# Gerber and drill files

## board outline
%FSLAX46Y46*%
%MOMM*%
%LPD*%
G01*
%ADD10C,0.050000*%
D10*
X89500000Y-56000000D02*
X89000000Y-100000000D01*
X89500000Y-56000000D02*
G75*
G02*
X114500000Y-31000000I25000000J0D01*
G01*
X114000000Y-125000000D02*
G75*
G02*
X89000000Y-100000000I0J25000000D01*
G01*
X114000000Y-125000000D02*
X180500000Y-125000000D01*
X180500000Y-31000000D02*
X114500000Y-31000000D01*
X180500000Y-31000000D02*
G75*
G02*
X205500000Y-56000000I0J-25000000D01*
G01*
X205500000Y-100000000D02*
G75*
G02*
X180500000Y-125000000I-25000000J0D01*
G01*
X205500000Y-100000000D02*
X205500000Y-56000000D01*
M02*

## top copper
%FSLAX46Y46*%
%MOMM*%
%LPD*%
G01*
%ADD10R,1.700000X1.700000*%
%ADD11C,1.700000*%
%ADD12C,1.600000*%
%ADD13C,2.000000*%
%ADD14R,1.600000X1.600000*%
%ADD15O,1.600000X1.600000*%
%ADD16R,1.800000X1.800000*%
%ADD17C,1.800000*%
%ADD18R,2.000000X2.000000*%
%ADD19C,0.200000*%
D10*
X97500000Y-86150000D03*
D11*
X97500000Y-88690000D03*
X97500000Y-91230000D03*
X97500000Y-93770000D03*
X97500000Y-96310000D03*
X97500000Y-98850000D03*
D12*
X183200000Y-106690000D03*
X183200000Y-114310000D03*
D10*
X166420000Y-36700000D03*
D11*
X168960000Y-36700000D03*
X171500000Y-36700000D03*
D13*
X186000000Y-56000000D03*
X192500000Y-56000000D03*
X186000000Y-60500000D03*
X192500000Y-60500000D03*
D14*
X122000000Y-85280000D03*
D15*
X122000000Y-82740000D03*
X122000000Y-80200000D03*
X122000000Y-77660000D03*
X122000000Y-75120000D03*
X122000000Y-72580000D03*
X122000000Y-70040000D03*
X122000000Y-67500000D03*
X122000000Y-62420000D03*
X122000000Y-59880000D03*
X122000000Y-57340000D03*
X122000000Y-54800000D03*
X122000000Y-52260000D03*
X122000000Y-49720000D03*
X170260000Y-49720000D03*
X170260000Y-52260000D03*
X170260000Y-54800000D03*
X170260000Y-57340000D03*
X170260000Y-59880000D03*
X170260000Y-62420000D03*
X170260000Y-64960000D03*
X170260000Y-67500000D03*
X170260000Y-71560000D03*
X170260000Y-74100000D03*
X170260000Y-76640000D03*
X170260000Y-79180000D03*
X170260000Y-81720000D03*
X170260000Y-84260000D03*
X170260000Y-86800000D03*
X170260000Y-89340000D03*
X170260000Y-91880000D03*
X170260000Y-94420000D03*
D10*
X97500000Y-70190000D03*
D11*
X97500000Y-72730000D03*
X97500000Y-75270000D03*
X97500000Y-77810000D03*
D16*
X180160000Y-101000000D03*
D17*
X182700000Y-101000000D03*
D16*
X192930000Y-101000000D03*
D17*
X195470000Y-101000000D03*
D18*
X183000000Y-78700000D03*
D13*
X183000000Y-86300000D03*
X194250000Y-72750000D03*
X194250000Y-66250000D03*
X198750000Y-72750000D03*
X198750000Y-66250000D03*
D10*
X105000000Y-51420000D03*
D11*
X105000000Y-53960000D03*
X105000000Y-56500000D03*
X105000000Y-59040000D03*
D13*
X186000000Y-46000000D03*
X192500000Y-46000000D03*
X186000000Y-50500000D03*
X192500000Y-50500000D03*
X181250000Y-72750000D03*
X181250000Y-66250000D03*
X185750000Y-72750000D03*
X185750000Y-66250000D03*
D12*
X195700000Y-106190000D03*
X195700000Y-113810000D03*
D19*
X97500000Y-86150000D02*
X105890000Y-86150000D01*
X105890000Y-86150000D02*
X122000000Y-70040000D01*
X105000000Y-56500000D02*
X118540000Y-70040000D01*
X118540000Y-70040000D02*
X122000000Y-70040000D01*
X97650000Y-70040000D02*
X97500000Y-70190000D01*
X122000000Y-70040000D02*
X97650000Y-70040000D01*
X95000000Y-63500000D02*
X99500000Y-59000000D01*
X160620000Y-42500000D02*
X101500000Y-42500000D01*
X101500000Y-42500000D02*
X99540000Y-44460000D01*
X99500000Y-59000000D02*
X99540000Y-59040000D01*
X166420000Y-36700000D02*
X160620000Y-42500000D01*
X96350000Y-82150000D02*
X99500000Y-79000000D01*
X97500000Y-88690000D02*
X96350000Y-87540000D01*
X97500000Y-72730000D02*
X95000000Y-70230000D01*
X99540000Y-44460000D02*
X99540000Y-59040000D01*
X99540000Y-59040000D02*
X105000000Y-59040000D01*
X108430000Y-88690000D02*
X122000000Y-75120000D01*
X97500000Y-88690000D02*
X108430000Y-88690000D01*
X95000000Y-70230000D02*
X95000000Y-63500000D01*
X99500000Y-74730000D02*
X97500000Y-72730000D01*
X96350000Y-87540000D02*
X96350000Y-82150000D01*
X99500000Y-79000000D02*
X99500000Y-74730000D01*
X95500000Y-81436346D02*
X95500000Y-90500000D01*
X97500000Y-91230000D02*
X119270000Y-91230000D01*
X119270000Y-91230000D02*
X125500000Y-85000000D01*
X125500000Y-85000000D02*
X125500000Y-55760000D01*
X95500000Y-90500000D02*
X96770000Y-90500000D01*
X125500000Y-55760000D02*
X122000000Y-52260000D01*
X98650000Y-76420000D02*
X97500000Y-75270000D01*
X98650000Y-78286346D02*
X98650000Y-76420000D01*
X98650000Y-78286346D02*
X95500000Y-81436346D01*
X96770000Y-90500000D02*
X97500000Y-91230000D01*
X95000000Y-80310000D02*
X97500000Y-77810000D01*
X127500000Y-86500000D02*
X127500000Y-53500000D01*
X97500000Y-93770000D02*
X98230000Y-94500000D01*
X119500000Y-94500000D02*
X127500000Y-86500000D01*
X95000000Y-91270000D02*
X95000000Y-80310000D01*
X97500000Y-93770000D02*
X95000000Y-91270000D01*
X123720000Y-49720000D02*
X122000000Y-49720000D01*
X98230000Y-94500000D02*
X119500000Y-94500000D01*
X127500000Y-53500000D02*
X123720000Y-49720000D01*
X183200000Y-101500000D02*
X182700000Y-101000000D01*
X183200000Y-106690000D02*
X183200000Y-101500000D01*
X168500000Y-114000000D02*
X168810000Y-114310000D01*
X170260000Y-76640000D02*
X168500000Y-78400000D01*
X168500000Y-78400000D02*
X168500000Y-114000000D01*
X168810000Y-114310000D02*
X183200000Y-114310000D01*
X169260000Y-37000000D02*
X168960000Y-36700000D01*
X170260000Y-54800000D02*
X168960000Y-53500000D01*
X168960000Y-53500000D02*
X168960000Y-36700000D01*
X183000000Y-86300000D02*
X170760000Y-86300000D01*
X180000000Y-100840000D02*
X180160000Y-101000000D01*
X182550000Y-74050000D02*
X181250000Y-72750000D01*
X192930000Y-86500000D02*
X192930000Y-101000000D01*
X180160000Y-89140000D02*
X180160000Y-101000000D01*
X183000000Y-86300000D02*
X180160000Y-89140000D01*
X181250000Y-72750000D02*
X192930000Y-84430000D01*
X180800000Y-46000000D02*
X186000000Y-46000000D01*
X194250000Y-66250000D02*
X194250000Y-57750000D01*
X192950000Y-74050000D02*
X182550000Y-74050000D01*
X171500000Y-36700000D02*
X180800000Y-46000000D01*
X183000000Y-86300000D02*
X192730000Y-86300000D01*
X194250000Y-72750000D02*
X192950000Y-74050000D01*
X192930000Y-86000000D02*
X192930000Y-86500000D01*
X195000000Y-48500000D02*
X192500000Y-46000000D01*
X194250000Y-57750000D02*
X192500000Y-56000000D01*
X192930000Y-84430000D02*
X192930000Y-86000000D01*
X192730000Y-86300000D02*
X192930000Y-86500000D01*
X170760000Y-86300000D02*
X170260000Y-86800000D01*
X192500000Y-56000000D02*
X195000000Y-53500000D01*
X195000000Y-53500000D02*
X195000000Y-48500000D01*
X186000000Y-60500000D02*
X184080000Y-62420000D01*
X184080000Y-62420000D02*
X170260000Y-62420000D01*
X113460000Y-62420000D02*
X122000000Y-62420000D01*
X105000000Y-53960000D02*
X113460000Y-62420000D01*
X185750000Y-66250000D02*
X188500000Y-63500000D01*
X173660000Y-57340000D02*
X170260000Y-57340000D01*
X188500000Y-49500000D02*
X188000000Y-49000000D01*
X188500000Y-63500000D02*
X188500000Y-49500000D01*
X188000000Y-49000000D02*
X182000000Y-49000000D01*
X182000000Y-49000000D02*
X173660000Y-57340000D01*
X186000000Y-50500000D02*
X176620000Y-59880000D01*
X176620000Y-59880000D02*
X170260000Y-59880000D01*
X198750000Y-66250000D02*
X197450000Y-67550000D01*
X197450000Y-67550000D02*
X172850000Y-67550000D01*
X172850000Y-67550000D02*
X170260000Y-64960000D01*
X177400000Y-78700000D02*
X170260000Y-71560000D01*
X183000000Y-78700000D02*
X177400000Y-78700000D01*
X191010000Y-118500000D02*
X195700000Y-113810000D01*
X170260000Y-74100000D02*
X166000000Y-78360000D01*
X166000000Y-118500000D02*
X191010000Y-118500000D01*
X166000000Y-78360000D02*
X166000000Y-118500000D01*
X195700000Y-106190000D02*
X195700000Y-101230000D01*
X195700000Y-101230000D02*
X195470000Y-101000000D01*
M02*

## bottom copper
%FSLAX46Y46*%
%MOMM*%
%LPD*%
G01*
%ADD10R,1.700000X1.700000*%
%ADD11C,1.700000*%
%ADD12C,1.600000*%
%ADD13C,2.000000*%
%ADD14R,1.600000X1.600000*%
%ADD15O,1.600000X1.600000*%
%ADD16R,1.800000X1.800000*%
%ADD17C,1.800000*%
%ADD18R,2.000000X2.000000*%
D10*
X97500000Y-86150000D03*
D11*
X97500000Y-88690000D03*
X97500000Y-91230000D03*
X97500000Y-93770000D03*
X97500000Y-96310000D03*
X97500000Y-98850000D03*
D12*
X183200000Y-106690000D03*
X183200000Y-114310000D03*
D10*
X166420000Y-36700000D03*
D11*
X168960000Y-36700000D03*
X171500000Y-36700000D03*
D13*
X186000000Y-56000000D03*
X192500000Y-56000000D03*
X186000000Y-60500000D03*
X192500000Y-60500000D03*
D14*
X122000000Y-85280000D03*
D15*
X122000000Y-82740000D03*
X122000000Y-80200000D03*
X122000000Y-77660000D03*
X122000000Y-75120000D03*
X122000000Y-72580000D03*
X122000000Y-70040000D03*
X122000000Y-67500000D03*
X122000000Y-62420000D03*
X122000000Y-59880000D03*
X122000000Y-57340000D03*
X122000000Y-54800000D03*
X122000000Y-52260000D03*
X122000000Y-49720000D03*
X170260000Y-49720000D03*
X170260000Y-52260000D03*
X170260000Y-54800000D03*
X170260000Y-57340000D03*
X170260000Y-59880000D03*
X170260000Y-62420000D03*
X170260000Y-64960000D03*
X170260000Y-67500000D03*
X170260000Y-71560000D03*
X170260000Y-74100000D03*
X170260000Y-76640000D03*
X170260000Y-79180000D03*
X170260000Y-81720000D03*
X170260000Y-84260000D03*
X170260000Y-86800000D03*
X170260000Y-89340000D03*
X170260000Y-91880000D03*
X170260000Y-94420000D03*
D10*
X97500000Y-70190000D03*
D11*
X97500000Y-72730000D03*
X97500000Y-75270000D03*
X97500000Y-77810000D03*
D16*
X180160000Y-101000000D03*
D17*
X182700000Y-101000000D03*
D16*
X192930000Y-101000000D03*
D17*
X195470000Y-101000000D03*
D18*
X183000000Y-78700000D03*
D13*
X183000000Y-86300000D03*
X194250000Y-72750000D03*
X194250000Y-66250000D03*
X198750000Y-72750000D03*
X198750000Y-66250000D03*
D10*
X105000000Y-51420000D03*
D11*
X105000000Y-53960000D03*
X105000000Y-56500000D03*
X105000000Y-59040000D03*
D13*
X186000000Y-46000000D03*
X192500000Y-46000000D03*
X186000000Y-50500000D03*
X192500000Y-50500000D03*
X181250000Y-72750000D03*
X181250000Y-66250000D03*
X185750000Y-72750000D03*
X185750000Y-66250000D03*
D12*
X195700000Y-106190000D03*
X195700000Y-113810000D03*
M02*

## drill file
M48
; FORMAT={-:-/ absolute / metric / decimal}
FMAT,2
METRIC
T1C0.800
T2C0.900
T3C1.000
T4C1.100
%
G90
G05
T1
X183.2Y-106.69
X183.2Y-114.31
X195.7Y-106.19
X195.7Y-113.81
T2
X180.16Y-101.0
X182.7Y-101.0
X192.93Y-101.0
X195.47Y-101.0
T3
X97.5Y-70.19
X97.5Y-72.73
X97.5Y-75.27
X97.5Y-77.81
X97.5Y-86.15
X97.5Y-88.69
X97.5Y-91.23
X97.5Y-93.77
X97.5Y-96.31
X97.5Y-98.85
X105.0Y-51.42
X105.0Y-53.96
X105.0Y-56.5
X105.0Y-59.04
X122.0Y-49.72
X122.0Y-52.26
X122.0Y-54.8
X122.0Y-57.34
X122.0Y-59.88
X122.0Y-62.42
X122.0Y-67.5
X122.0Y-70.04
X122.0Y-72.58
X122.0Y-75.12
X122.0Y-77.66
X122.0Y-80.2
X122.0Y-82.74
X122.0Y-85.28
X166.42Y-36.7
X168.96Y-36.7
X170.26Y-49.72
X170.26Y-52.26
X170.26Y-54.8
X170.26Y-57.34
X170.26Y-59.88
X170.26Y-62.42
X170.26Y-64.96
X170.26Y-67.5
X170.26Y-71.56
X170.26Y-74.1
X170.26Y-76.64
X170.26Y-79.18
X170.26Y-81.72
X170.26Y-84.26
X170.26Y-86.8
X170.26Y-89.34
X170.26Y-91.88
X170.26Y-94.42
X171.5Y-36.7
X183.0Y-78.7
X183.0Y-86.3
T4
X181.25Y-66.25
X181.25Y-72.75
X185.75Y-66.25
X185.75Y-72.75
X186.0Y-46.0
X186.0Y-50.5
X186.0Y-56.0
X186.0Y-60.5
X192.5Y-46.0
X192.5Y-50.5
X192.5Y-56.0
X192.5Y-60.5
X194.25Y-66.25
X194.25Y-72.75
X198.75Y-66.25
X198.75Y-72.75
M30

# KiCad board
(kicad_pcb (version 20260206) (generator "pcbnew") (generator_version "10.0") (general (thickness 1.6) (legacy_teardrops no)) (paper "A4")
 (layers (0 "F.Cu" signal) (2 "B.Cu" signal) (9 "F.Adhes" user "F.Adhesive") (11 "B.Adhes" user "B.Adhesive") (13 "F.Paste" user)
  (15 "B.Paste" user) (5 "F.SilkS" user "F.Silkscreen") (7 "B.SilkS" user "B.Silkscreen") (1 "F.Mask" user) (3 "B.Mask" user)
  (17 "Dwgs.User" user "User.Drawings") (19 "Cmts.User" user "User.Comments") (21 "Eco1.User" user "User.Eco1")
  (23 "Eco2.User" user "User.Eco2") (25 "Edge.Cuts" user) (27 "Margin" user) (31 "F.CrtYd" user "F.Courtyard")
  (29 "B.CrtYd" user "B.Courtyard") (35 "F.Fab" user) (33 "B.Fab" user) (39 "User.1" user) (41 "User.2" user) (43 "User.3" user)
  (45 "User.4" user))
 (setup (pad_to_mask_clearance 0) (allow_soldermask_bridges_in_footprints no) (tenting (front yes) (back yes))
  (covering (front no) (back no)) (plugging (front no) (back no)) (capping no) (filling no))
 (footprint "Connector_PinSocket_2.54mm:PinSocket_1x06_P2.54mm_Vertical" (layer "F.Cu") (at 97.5 86.15)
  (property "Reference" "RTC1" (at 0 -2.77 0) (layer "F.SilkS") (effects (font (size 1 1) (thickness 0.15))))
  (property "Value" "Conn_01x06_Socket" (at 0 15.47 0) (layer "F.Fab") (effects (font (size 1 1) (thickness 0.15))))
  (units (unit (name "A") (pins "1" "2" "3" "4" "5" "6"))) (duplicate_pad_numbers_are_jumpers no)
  (pad "1" thru_hole rect (at 0 0) (size 1.7 1.7) (drill 1) (layers "*.Cu" "*.Mask") (remove_unused_layers no) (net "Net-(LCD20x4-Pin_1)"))
  (pad "2" thru_hole circle (at 0 2.54) (size 1.7 1.7) (drill 1) (layers "*.Cu" "*.Mask") (remove_unused_layers no) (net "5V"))
  (pad "3" thru_hole circle (at 0 5.08) (size 1.7 1.7) (drill 1) (layers "*.Cu" "*.Mask") (remove_unused_layers no)
   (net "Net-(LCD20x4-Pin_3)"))
  (pad "4" thru_hole circle (at 0 7.62) (size 1.7 1.7) (drill 1) (layers "*.Cu" "*.Mask") (remove_unused_layers no)
   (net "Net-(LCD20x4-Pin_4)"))
  (pad "5" thru_hole circle (at 0 10.16) (size 1.7 1.7) (drill 1) (layers "*.Cu" "*.Mask") (remove_unused_layers no)
   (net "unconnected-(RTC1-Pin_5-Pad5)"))
  (pad "6" thru_hole circle (at 0 12.7) (size 1.7 1.7) (drill 1) (layers "*.Cu" "*.Mask") (remove_unused_layers no)
   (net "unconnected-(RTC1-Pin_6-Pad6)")))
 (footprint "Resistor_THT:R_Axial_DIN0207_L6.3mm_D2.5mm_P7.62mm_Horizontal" (layer "F.Cu") (at 183.2 106.69 -90)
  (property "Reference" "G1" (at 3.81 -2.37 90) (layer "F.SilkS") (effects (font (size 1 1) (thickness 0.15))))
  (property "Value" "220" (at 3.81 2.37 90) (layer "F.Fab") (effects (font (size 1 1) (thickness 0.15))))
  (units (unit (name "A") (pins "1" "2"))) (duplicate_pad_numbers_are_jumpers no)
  (pad "1" thru_hole circle (at 0 0 270) (size 1.6 1.6) (drill 0.8) (layers "*.Cu" "*.Mask") (remove_unused_layers no)
   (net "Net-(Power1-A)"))
  (pad "2" thru_hole circle (at 7.62 0 270) (size 1.6 1.6) (drill 0.8) (layers "*.Cu" "*.Mask") (remove_unused_layers no)
   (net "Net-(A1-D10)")))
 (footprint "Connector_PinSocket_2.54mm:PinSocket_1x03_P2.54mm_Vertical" (layer "F.Cu") (at 166.42 36.7 90)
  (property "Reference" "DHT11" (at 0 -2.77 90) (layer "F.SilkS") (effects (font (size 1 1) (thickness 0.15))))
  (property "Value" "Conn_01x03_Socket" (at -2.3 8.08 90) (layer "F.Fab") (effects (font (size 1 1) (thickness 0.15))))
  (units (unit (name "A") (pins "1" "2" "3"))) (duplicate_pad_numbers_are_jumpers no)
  (pad "1" thru_hole rect (at 0 0 90) (size 1.7 1.7) (drill 1) (layers "*.Cu" "*.Mask") (remove_unused_layers no) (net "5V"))
  (pad "2" thru_hole circle (at 0 2.54 90) (size 1.7 1.7) (drill 1) (layers "*.Cu" "*.Mask") (remove_unused_layers no) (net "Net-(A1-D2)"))
  (pad "3" thru_hole circle (at 0 5.08 90) (size 1.7 1.7) (drill 1) (layers "*.Cu" "*.Mask") (remove_unused_layers no)
   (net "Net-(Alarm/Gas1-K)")))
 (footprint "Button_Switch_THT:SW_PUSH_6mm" (layer "F.Cu") (at 186 56)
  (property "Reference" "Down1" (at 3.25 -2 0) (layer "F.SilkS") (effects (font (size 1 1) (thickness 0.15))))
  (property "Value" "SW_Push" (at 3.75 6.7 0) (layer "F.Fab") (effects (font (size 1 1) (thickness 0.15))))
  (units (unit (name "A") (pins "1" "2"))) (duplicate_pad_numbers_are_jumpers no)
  (pad "1" thru_hole circle (at 0 0 90) (size 2 2) (drill 1.1) (layers "*.Cu" "*.Mask") (remove_unused_layers no) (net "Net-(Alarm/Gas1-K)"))
  (pad "1" thru_hole circle (at 6.5 0 90) (size 2 2) (drill 1.1) (layers "*.Cu" "*.Mask") (remove_unused_layers no)
   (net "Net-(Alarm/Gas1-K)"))
  (pad "2" thru_hole circle (at 0 4.5 90) (size 2 2) (drill 1.1) (layers "*.Cu" "*.Mask") (remove_unused_layers no) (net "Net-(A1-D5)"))
  (pad "2" thru_hole circle (at 6.5 4.5 90) (size 2 2) (drill 1.1) (layers "*.Cu" "*.Mask") (remove_unused_layers no) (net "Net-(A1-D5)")))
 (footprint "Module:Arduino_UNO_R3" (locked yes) (layer "F.Cu") (at 122 85.28 90)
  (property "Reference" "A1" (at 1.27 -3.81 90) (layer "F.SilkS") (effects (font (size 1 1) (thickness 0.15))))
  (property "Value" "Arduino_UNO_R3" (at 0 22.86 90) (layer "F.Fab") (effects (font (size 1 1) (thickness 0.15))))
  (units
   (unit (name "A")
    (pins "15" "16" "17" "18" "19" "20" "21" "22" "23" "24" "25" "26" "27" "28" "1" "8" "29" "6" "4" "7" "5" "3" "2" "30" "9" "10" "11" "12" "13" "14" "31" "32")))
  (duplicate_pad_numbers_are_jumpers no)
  (pad "1" thru_hole rect (at 0 0 180) (size 1.6 1.6) (drill 1) (layers "*.Cu" "*.Mask") (remove_unused_layers no)
   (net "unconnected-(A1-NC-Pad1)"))
  (pad "2" thru_hole oval (at 2.54 0 180) (size 1.6 1.6) (drill 1) (layers "*.Cu" "*.Mask") (remove_unused_layers no)
   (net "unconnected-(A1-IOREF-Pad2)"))
  (pad "3" thru_hole oval (at 5.08 0 180) (size 1.6 1.6) (drill 1) (layers "*.Cu" "*.Mask") (remove_unused_layers no)
   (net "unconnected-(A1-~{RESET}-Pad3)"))
  (pad "4" thru_hole oval (at 7.62 0 180) (size 1.6 1.6) (drill 1) (layers "*.Cu" "*.Mask") (remove_unused_layers no)
   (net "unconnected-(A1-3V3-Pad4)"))
  (pad "5" thru_hole oval (at 10.16 0 180) (size 1.6 1.6) (drill 1) (layers "*.Cu" "*.Mask") (remove_unused_layers no) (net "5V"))
  (pad "6" thru_hole oval (at 12.7 0 180) (size 1.6 1.6) (drill 1) (layers "*.Cu" "*.Mask") (remove_unused_layers no) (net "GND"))
  (pad "7" thru_hole oval (at 15.24 0 180) (size 1.6 1.6) (drill 1) (layers "*.Cu" "*.Mask") (remove_unused_layers no)
   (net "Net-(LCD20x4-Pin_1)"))
  (pad "8" thru_hole oval (at 17.78 0 180) (size 1.6 1.6) (drill 1) (layers "*.Cu" "*.Mask") (remove_unused_layers no)
   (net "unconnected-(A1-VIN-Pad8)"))
  (pad "9" thru_hole oval (at 22.86 0 180) (size 1.6 1.6) (drill 1) (layers "*.Cu" "*.Mask") (remove_unused_layers no) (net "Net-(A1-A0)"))
  (pad "10" thru_hole oval (at 25.4 0 180) (size 1.6 1.6) (drill 1) (layers "*.Cu" "*.Mask") (remove_unused_layers no)
   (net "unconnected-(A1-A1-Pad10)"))
  (pad "11" thru_hole oval (at 27.94 0 180) (size 1.6 1.6) (drill 1) (layers "*.Cu" "*.Mask") (remove_unused_layers no)
   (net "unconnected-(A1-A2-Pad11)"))
  (pad "12" thru_hole oval (at 30.48 0 180) (size 1.6 1.6) (drill 1) (layers "*.Cu" "*.Mask") (remove_unused_layers no)
   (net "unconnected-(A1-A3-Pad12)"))
  (pad "13" thru_hole oval (at 33.02 0 180) (size 1.6 1.6) (drill 1) (layers "*.Cu" "*.Mask") (remove_unused_layers no)
   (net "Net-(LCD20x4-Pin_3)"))
  (pad "14" thru_hole oval (at 35.56 0 180) (size 1.6 1.6) (drill 1) (layers "*.Cu" "*.Mask") (remove_unused_layers no)
   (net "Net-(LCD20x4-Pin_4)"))
  (pad "15" thru_hole oval (at 35.56 48.26 180) (size 1.6 1.6) (drill 1) (layers "*.Cu" "*.Mask") (remove_unused_layers no)
   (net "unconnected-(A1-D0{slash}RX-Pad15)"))
  (pad "16" thru_hole oval (at 33.02 48.26 180) (size 1.6 1.6) (drill 1) (layers "*.Cu" "*.Mask") (remove_unused_layers no)
   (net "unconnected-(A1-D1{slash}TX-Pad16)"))
  (pad "17" thru_hole oval (at 30.48 48.26 180) (size 1.6 1.6) (drill 1) (layers "*.Cu" "*.Mask") (remove_unused_layers no)
   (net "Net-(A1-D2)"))
  (pad "18" thru_hole oval (at 27.94 48.26 180) (size 1.6 1.6) (drill 1) (layers "*.Cu" "*.Mask") (remove_unused_layers no)
   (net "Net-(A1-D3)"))
  (pad "19" thru_hole oval (at 25.4 48.26 180) (size 1.6 1.6) (drill 1) (layers "*.Cu" "*.Mask") (remove_unused_layers no)
   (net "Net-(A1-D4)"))
  (pad "20" thru_hole oval (at 22.86 48.26 180) (size 1.6 1.6) (drill 1) (layers "*.Cu" "*.Mask") (remove_unused_layers no)
   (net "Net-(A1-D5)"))
  (pad "21" thru_hole oval (at 20.32 48.26 180) (size 1.6 1.6) (drill 1) (layers "*.Cu" "*.Mask") (remove_unused_layers no)
   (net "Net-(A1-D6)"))
  (pad "22" thru_hole oval (at 17.78 48.26 180) (size 1.6 1.6) (drill 1) (layers "*.Cu" "*.Mask") (remove_unused_layers no)
   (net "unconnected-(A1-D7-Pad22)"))
  (pad "23" thru_hole oval (at 13.72 48.26 180) (size 1.6 1.6) (drill 1) (layers "*.Cu" "*.Mask") (remove_unused_layers no)
   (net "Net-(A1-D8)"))
  (pad "24" thru_hole oval (at 11.18 48.26 180) (size 1.6 1.6) (drill 1) (layers "*.Cu" "*.Mask") (remove_unused_layers no)
   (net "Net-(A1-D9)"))
  (pad "25" thru_hole oval (at 8.64 48.26 180) (size 1.6 1.6) (drill 1) (layers "*.Cu" "*.Mask") (remove_unused_layers no)
   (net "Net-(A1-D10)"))
  (pad "26" thru_hole oval (at 6.1 48.26 180) (size 1.6 1.6) (drill 1) (layers "*.Cu" "*.Mask") (remove_unused_layers no)
   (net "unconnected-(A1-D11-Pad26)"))
  (pad "27" thru_hole oval (at 3.56 48.26 180) (size 1.6 1.6) (drill 1) (layers "*.Cu" "*.Mask") (remove_unused_layers no)
   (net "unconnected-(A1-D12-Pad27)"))
  (pad "28" thru_hole oval (at 1.02 48.26 180) (size 1.6 1.6) (drill 1) (layers "*.Cu" "*.Mask") (remove_unused_layers no)
   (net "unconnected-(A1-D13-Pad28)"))
  (pad "29" thru_hole oval (at -1.52 48.26 180) (size 1.6 1.6) (drill 1) (layers "*.Cu" "*.Mask") (remove_unused_layers no)
   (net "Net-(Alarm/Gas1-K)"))
  (pad "30" thru_hole oval (at -4.06 48.26 180) (size 1.6 1.6) (drill 1) (layers "*.Cu" "*.Mask") (remove_unused_layers no)
   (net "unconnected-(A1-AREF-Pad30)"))
  (pad "31" thru_hole oval (at -6.6 48.26 180) (size 1.6 1.6) (drill 1) (layers "*.Cu" "*.Mask") (remove_unused_layers no)
   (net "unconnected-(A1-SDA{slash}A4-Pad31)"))
  (pad "32" thru_hole oval (at -9.14 48.26 180) (size 1.6 1.6) (drill 1) (layers "*.Cu" "*.Mask") (remove_unused_layers no)
   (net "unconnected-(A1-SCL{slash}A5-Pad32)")))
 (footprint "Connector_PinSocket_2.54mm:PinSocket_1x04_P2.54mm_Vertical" (layer "F.Cu") (at 97.5 70.19)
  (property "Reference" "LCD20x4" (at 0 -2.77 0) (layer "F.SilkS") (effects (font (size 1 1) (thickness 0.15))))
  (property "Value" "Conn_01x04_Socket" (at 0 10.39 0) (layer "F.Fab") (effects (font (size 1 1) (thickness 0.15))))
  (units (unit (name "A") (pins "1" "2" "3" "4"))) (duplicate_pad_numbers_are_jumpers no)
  (pad "1" thru_hole rect (at 0 0) (size 1.7 1.7) (drill 1) (layers "*.Cu" "*.Mask") (remove_unused_layers no) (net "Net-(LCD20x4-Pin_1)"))
  (pad "2" thru_hole circle (at 0 2.54) (size 1.7 1.7) (drill 1) (layers "*.Cu" "*.Mask") (remove_unused_layers no) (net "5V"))
  (pad "3" thru_hole circle (at 0 5.08) (size 1.7 1.7) (drill 1) (layers "*.Cu" "*.Mask") (remove_unused_layers no)
   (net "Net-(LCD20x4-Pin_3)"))
  (pad "4" thru_hole circle (at 0 7.62) (size 1.7 1.7) (drill 1) (layers "*.Cu" "*.Mask") (remove_unused_layers no)
   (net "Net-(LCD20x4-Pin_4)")))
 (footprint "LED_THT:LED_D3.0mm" (layer "F.Cu") (at 180.16 101)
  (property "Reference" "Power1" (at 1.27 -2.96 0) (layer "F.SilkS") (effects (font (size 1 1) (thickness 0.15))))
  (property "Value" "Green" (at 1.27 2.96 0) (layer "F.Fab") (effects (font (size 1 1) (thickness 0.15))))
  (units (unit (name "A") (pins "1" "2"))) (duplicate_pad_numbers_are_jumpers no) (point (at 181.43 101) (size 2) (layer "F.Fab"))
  (pad "1" thru_hole rect (at 0 0) (size 1.8 1.8) (drill 0.9) (layers "*.Cu" "*.Mask") (remove_unused_layers no) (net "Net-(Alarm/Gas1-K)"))
  (pad "2" thru_hole circle (at 2.54 0) (size 1.8 1.8) (drill 0.9) (layers "*.Cu" "*.Mask") (remove_unused_layers no) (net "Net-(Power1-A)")))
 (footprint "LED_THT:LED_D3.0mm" (layer "F.Cu") (at 192.93 101)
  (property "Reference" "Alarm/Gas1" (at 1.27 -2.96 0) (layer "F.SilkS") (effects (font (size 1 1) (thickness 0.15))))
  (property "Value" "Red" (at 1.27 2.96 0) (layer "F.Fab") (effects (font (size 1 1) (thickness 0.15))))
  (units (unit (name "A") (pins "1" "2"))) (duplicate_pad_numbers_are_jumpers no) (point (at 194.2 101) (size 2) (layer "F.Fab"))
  (pad "1" thru_hole rect (at 0 0) (size 1.8 1.8) (drill 0.9) (layers "*.Cu" "*.Mask") (remove_unused_layers no) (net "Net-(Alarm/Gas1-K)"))
  (pad "2" thru_hole circle (at 2.54 0) (size 1.8 1.8) (drill 0.9) (layers "*.Cu" "*.Mask") (remove_unused_layers no)
   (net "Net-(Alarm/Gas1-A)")))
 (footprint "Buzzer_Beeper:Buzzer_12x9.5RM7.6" (layer "F.Cu") (at 183 78.7 -90)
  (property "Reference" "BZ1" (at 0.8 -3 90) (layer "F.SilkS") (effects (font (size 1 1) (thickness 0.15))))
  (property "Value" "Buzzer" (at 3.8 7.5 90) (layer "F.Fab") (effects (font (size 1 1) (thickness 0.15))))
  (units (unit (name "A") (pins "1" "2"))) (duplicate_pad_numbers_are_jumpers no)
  (pad "1" thru_hole rect (at 0 0 270) (size 2 2) (drill 1) (layers "*.Cu" "*.Mask") (remove_unused_layers no) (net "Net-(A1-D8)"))
  (pad "2" thru_hole circle (at 7.6 0 270) (size 2 2) (drill 1) (layers "*.Cu" "*.Mask") (remove_unused_layers no)
   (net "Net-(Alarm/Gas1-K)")))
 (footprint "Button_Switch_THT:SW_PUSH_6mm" (layer "F.Cu") (at 194.25 72.75 90)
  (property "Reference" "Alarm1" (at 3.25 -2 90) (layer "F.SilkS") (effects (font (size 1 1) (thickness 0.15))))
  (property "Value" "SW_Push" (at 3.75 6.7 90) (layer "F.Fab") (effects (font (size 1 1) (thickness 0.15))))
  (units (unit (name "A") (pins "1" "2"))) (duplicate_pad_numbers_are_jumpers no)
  (pad "1" thru_hole circle (at 0 0 180) (size 2 2) (drill 1.1) (layers "*.Cu" "*.Mask") (remove_unused_layers no)
   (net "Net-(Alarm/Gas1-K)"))
  (pad "1" thru_hole circle (at 6.5 0 180) (size 2 2) (drill 1.1) (layers "*.Cu" "*.Mask") (remove_unused_layers no)
   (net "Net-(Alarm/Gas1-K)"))
  (pad "2" thru_hole circle (at 0 4.5 180) (size 2 2) (drill 1.1) (layers "*.Cu" "*.Mask") (remove_unused_layers no) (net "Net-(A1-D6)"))
  (pad "2" thru_hole circle (at 6.5 4.5 180) (size 2 2) (drill 1.1) (layers "*.Cu" "*.Mask") (remove_unused_layers no) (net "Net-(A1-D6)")))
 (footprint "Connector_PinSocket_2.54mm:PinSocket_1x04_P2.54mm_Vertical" (layer "F.Cu") (at 105 51.42)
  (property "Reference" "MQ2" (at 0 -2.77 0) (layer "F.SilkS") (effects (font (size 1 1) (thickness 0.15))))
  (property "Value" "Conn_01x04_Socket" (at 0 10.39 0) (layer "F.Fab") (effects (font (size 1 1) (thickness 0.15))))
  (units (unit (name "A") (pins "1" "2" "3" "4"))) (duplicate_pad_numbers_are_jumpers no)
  (pad "1" thru_hole rect (at 0 0) (size 1.7 1.7) (drill 1) (layers "*.Cu" "*.Mask") (remove_unused_layers no)
   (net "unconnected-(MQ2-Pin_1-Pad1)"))
  (pad "2" thru_hole circle (at 0 2.54) (size 1.7 1.7) (drill 1) (layers "*.Cu" "*.Mask") (remove_unused_layers no) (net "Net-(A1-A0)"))
  (pad "3" thru_hole circle (at 0 5.08) (size 1.7 1.7) (drill 1) (layers "*.Cu" "*.Mask") (remove_unused_layers no)
   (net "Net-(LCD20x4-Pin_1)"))
  (pad "4" thru_hole circle (at 0 7.62) (size 1.7 1.7) (drill 1) (layers "*.Cu" "*.Mask") (remove_unused_layers no) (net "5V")))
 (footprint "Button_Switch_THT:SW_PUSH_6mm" (layer "F.Cu") (at 186 46)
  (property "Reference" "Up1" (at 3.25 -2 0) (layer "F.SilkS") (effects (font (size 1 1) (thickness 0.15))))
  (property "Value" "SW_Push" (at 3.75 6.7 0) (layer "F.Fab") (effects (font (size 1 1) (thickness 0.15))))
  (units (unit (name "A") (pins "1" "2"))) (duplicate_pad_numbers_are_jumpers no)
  (pad "1" thru_hole circle (at 0 0 90) (size 2 2) (drill 1.1) (layers "*.Cu" "*.Mask") (remove_unused_layers no) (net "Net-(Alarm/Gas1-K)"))
  (pad "1" thru_hole circle (at 6.5 0 90) (size 2 2) (drill 1.1) (layers "*.Cu" "*.Mask") (remove_unused_layers no)
   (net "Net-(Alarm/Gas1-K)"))
  (pad "2" thru_hole circle (at 0 4.5 90) (size 2 2) (drill 1.1) (layers "*.Cu" "*.Mask") (remove_unused_layers no) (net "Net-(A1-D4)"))
  (pad "2" thru_hole circle (at 6.5 4.5 90) (size 2 2) (drill 1.1) (layers "*.Cu" "*.Mask") (remove_unused_layers no) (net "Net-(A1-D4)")))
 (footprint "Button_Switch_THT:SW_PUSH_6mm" (layer "F.Cu") (at 181.25 72.75 90)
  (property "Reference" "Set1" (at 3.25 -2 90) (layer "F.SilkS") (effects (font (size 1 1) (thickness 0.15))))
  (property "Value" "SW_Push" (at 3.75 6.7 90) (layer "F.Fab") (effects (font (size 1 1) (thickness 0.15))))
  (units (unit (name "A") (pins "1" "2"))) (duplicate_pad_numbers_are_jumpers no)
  (pad "1" thru_hole circle (at 0 0 180) (size 2 2) (drill 1.1) (layers "*.Cu" "*.Mask") (remove_unused_layers no)
   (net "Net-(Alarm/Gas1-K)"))
  (pad "1" thru_hole circle (at 6.5 0 180) (size 2 2) (drill 1.1) (layers "*.Cu" "*.Mask") (remove_unused_layers no)
   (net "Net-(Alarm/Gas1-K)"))
  (pad "2" thru_hole circle (at 0 4.5 180) (size 2 2) (drill 1.1) (layers "*.Cu" "*.Mask") (remove_unused_layers no) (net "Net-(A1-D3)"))
  (pad "2" thru_hole circle (at 6.5 4.5 180) (size 2 2) (drill 1.1) (layers "*.Cu" "*.Mask") (remove_unused_layers no) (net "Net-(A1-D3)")))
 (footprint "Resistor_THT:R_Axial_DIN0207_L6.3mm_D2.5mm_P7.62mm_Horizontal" (layer "F.Cu") (at 195.7 106.19 -90)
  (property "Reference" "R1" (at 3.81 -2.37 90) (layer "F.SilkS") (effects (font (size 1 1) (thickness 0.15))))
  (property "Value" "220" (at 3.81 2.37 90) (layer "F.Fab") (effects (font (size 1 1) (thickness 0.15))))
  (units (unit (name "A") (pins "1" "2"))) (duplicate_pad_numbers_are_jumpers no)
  (pad "1" thru_hole circle (at 0 0 270) (size 1.6 1.6) (drill 0.8) (layers "*.Cu" "*.Mask") (remove_unused_layers no)
   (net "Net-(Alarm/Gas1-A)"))
  (pad "2" thru_hole circle (at 7.62 0 270) (size 1.6 1.6) (drill 0.8) (layers "*.Cu" "*.Mask") (remove_unused_layers no)
   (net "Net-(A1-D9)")))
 (gr_line (start 89.5 56) (end 89 100) (stroke (width 0.05) (type default)) (layer "Edge.Cuts"))
 (gr_arc (start 89.5 56) (mid 96.82233 38.32233) (end 114.5 31) (stroke (width 0.05) (type default)) (layer "Edge.Cuts"))
 (gr_arc (start 114 125) (mid 96.32233 117.67767) (end 89 100) (stroke (width 0.05) (type default)) (layer "Edge.Cuts"))
 (gr_line (start 114 125) (end 180.5 125) (stroke (width 0.05) (type default)) (layer "Edge.Cuts"))
 (gr_line (start 180.5 31) (end 114.5 31) (stroke (width 0.05) (type default)) (layer "Edge.Cuts"))
 (gr_arc (start 180.5 31) (mid 198.17767 38.32233) (end 205.5 56) (stroke (width 0.05) (type default)) (layer "Edge.Cuts"))
 (gr_arc (start 205.5 100) (mid 198.17767 117.67767) (end 180.5 125) (stroke (width 0.05) (type default)) (layer "Edge.Cuts"))
 (gr_line (start 205.5 100) (end 205.5 56) (stroke (width 0.05) (type default)) (layer "Edge.Cuts"))
 (segment (start 97.5 86.15) (end 105.89 86.15) (width 0.2) (layer "F.Cu") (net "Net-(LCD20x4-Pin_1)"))
 (segment (start 105.89 86.15) (end 122 70.04) (width 0.2) (layer "F.Cu") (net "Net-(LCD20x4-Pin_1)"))
 (segment (start 105 56.5) (end 118.54 70.04) (width 0.2) (layer "F.Cu") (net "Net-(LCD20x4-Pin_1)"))
 (segment (start 118.54 70.04) (end 122 70.04) (width 0.2) (layer "F.Cu") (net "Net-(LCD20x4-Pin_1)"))
 (segment (start 97.65 70.04) (end 97.5 70.19) (width 0.2) (layer "F.Cu") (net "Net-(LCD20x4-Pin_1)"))
 (segment (start 122 70.04) (end 97.65 70.04) (width 0.2) (layer "F.Cu") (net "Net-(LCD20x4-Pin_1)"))
 (segment (start 95 63.5) (end 99.5 59) (width 0.2) (layer "F.Cu") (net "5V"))
 (segment (start 160.62 42.5) (end 101.5 42.5) (width 0.2) (layer "F.Cu") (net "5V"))
 (segment (start 101.5 42.5) (end 99.54 44.46) (width 0.2) (layer "F.Cu") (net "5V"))
 (segment (start 99.5 59) (end 99.54 59.04) (width 0.2) (layer "F.Cu") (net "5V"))
 (segment (start 166.42 36.7) (end 160.62 42.5) (width 0.2) (layer "F.Cu") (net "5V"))
 (segment (start 96.35 82.15) (end 99.5 79) (width 0.2) (layer "F.Cu") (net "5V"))
 (segment (start 97.5 88.69) (end 96.35 87.54) (width 0.2) (layer "F.Cu") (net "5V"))
 (segment (start 97.5 72.73) (end 95 70.23) (width 0.2) (layer "F.Cu") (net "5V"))
 (segment (start 99.54 44.46) (end 99.54 59.04) (width 0.2) (layer "F.Cu") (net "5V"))
 (segment (start 99.54 59.04) (end 105 59.04) (width 0.2) (layer "F.Cu") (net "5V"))
 (segment (start 108.43 88.69) (end 122 75.12) (width 0.2) (layer "F.Cu") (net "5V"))
 (segment (start 97.5 88.69) (end 108.43 88.69) (width 0.2) (layer "F.Cu") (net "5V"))
 (segment (start 95 70.23) (end 95 63.5) (width 0.2) (layer "F.Cu") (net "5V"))
 (segment (start 99.5 74.73) (end 97.5 72.73) (width 0.2) (layer "F.Cu") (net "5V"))
 (segment (start 96.35 87.54) (end 96.35 82.15) (width 0.2) (layer "F.Cu") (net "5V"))
 (segment (start 99.5 79) (end 99.5 74.73) (width 0.2) (layer "F.Cu") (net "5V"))
 (segment (start 95.5 81.436346) (end 95.5 90.5) (width 0.2) (layer "F.Cu") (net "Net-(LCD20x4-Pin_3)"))
 (segment (start 97.5 91.23) (end 119.27 91.23) (width 0.2) (layer "F.Cu") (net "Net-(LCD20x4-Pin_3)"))
 (segment (start 119.27 91.23) (end 125.5 85) (width 0.2) (layer "F.Cu") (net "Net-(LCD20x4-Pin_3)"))
 (segment (start 125.5 85) (end 125.5 55.76) (width 0.2) (layer "F.Cu") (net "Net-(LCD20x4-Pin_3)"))
 (segment (start 95.5 90.5) (end 96.77 90.5) (width 0.2) (layer "F.Cu") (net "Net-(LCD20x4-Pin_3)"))
 (segment (start 125.5 55.76) (end 122 52.26) (width 0.2) (layer "F.Cu") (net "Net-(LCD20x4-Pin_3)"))
 (segment (start 98.65 76.42) (end 97.5 75.27) (width 0.2) (layer "F.Cu") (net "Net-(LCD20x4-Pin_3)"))
 (segment (start 98.65 78.286346) (end 98.65 76.42) (width 0.2) (layer "F.Cu") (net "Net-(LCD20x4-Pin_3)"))
 (segment (start 98.65 78.286346) (end 95.5 81.436346) (width 0.2) (layer "F.Cu") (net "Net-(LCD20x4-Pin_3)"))
 (segment (start 96.77 90.5) (end 97.5 91.23) (width 0.2) (layer "F.Cu") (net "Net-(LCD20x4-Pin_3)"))
 (segment (start 95 80.31) (end 97.5 77.81) (width 0.2) (layer "F.Cu") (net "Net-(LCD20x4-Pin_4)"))
 (segment (start 127.5 86.5) (end 127.5 53.5) (width 0.2) (layer "F.Cu") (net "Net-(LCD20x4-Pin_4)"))
 (segment (start 97.5 93.77) (end 98.23 94.5) (width 0.2) (layer "F.Cu") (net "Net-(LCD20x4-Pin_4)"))
 (segment (start 119.5 94.5) (end 127.5 86.5) (width 0.2) (layer "F.Cu") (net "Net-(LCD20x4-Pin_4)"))
 (segment (start 95 91.27) (end 95 80.31) (width 0.2) (layer "F.Cu") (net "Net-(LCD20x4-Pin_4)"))
 (segment (start 97.5 93.77) (end 95 91.27) (width 0.2) (layer "F.Cu") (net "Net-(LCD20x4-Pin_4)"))
 (segment (start 123.72 49.72) (end 122 49.72) (width 0.2) (layer "F.Cu") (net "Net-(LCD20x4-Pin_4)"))
 (segment (start 98.23 94.5) (end 119.5 94.5) (width 0.2) (layer "F.Cu") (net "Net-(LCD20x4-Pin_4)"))
 (segment (start 127.5 53.5) (end 123.72 49.72) (width 0.2) (layer "F.Cu") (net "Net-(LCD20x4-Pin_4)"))
 (segment (start 183.2 101.5) (end 182.7 101) (width 0.2) (layer "F.Cu") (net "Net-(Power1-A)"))
 (segment (start 183.2 106.69) (end 183.2 101.5) (width 0.2) (layer "F.Cu") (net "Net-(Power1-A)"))
 (segment (start 168.5 114) (end 168.81 114.31) (width 0.2) (layer "F.Cu") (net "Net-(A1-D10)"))
 (segment (start 170.26 76.64) (end 168.5 78.4) (width 0.2) (layer "F.Cu") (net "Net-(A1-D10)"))
 (segment (start 168.5 78.4) (end 168.5 114) (width 0.2) (layer "F.Cu") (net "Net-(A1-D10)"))
 (segment (start 168.81 114.31) (end 183.2 114.31) (width 0.2) (layer "F.Cu") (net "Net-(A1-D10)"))
 (segment (start 169.26 37) (end 168.96 36.7) (width 0.2) (layer "F.Cu") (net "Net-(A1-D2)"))
 (segment (start 170.26 54.8) (end 168.96 53.5) (width 0.2) (layer "F.Cu") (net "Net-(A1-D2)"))
 (segment (start 168.96 53.5) (end 168.96 36.7) (width 0.2) (layer "F.Cu") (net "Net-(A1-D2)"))
 (segment (start 183 86.3) (end 170.76 86.3) (width 0.2) (layer "F.Cu") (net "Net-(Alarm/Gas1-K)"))
 (segment (start 180 100.84) (end 180.16 101) (width 0.2) (layer "F.Cu") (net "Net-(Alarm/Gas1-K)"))
 (segment (start 182.55 74.05) (end 181.25 72.75) (width 0.2) (layer "F.Cu") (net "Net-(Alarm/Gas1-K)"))
 (segment (start 192.93 86.5) (end 192.93 101) (width 0.2) (layer "F.Cu") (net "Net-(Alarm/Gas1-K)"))
 (segment (start 180.16 89.14) (end 180.16 101) (width 0.2) (layer "F.Cu") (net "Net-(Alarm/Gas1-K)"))
 (segment (start 183 86.3) (end 180.16 89.14) (width 0.2) (layer "F.Cu") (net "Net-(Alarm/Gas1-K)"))
 (segment (start 181.25 72.75) (end 192.93 84.43) (width 0.2) (layer "F.Cu") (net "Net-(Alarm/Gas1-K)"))
 (segment (start 180.8 46) (end 186 46) (width 0.2) (layer "F.Cu") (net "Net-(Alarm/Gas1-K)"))
 (segment (start 194.25 66.25) (end 194.25 57.75) (width 0.2) (layer "F.Cu") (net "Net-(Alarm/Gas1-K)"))
 (segment (start 192.95 74.05) (end 182.55 74.05) (width 0.2) (layer "F.Cu") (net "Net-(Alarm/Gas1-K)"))
 (segment (start 171.5 36.7) (end 180.8 46) (width 0.2) (layer "F.Cu") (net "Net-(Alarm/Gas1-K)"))
 (segment (start 183 86.3) (end 192.73 86.3) (width 0.2) (layer "F.Cu") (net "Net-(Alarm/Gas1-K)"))
 (segment (start 194.25 72.75) (end 192.95 74.05) (width 0.2) (layer "F.Cu") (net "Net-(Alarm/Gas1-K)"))
 (segment (start 192.93 86) (end 192.93 86.5) (width 0.2) (layer "F.Cu") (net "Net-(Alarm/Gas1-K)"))
 (segment (start 195 48.5) (end 192.5 46) (width 0.2) (layer "F.Cu") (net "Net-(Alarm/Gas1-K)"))
 (segment (start 194.25 57.75) (end 192.5 56) (width 0.2) (layer "F.Cu") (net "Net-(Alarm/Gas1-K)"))
 (segment (start 192.93 84.43) (end 192.93 86) (width 0.2) (layer "F.Cu") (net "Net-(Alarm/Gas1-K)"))
 (segment (start 192.73 86.3) (end 192.93 86.5) (width 0.2) (layer "F.Cu") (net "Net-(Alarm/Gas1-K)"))
 (segment (start 170.76 86.3) (end 170.26 86.8) (width 0.2) (layer "F.Cu") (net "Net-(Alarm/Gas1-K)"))
 (segment (start 192.5 56) (end 195 53.5) (width 0.2) (layer "F.Cu") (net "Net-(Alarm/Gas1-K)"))
 (segment (start 195 53.5) (end 195 48.5) (width 0.2) (layer "F.Cu") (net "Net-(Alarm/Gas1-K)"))
 (segment (start 186 60.5) (end 184.08 62.42) (width 0.2) (layer "F.Cu") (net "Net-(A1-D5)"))
 (segment (start 184.08 62.42) (end 170.26 62.42) (width 0.2) (layer "F.Cu") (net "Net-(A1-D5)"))
 (segment (start 113.46 62.42) (end 122 62.42) (width 0.2) (layer "F.Cu") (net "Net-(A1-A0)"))
 (segment (start 105 53.96) (end 113.46 62.42) (width 0.2) (layer "F.Cu") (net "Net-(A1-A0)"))
 (segment (start 185.75 66.25) (end 188.5 63.5) (width 0.2) (layer "F.Cu") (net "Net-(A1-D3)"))
 (segment (start 173.66 57.34) (end 170.26 57.34) (width 0.2) (layer "F.Cu") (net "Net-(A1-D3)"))
 (segment (start 188.5 49.5) (end 188 49) (width 0.2) (layer "F.Cu") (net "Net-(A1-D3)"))
 (segment (start 188.5 63.5) (end 188.5 49.5) (width 0.2) (layer "F.Cu") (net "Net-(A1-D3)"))
 (segment (start 188 49) (end 182 49) (width 0.2) (layer "F.Cu") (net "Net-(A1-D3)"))
 (segment (start 182 49) (end 173.66 57.34) (width 0.2) (layer "F.Cu") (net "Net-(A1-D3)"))
 (segment (start 186 50.5) (end 176.62 59.88) (width 0.2) (layer "F.Cu") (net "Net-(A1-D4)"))
 (segment (start 176.62 59.88) (end 170.26 59.88) (width 0.2) (layer "F.Cu") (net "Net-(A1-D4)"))
 (segment (start 198.75 66.25) (end 197.45 67.55) (width 0.2) (layer "F.Cu") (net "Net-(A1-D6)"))
 (segment (start 197.45 67.55) (end 172.85 67.55) (width 0.2) (layer "F.Cu") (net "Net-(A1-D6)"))
 (segment (start 172.85 67.55) (end 170.26 64.96) (width 0.2) (layer "F.Cu") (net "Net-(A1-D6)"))
 (segment (start 177.4 78.7) (end 170.26 71.56) (width 0.2) (layer "F.Cu") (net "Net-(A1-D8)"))
 (segment (start 183 78.7) (end 177.4 78.7) (width 0.2) (layer "F.Cu") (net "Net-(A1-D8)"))
 (segment (start 191.01 118.5) (end 195.7 113.81) (width 0.2) (layer "F.Cu") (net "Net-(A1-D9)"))
 (segment (start 170.26 74.1) (end 166 78.36) (width 0.2) (layer "F.Cu") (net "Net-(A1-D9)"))
 (segment (start 166 118.5) (end 191.01 118.5) (width 0.2) (layer "F.Cu") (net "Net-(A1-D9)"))
 (segment (start 166 78.36) (end 166 118.5) (width 0.2) (layer "F.Cu") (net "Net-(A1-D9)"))
 (segment (start 195.7 106.19) (end 195.7 101.23) (width 0.2) (layer "F.Cu") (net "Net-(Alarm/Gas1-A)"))
 (segment (start 195.7 101.23) (end 195.47 101) (width 0.2) (layer "F.Cu") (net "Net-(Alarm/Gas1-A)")))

